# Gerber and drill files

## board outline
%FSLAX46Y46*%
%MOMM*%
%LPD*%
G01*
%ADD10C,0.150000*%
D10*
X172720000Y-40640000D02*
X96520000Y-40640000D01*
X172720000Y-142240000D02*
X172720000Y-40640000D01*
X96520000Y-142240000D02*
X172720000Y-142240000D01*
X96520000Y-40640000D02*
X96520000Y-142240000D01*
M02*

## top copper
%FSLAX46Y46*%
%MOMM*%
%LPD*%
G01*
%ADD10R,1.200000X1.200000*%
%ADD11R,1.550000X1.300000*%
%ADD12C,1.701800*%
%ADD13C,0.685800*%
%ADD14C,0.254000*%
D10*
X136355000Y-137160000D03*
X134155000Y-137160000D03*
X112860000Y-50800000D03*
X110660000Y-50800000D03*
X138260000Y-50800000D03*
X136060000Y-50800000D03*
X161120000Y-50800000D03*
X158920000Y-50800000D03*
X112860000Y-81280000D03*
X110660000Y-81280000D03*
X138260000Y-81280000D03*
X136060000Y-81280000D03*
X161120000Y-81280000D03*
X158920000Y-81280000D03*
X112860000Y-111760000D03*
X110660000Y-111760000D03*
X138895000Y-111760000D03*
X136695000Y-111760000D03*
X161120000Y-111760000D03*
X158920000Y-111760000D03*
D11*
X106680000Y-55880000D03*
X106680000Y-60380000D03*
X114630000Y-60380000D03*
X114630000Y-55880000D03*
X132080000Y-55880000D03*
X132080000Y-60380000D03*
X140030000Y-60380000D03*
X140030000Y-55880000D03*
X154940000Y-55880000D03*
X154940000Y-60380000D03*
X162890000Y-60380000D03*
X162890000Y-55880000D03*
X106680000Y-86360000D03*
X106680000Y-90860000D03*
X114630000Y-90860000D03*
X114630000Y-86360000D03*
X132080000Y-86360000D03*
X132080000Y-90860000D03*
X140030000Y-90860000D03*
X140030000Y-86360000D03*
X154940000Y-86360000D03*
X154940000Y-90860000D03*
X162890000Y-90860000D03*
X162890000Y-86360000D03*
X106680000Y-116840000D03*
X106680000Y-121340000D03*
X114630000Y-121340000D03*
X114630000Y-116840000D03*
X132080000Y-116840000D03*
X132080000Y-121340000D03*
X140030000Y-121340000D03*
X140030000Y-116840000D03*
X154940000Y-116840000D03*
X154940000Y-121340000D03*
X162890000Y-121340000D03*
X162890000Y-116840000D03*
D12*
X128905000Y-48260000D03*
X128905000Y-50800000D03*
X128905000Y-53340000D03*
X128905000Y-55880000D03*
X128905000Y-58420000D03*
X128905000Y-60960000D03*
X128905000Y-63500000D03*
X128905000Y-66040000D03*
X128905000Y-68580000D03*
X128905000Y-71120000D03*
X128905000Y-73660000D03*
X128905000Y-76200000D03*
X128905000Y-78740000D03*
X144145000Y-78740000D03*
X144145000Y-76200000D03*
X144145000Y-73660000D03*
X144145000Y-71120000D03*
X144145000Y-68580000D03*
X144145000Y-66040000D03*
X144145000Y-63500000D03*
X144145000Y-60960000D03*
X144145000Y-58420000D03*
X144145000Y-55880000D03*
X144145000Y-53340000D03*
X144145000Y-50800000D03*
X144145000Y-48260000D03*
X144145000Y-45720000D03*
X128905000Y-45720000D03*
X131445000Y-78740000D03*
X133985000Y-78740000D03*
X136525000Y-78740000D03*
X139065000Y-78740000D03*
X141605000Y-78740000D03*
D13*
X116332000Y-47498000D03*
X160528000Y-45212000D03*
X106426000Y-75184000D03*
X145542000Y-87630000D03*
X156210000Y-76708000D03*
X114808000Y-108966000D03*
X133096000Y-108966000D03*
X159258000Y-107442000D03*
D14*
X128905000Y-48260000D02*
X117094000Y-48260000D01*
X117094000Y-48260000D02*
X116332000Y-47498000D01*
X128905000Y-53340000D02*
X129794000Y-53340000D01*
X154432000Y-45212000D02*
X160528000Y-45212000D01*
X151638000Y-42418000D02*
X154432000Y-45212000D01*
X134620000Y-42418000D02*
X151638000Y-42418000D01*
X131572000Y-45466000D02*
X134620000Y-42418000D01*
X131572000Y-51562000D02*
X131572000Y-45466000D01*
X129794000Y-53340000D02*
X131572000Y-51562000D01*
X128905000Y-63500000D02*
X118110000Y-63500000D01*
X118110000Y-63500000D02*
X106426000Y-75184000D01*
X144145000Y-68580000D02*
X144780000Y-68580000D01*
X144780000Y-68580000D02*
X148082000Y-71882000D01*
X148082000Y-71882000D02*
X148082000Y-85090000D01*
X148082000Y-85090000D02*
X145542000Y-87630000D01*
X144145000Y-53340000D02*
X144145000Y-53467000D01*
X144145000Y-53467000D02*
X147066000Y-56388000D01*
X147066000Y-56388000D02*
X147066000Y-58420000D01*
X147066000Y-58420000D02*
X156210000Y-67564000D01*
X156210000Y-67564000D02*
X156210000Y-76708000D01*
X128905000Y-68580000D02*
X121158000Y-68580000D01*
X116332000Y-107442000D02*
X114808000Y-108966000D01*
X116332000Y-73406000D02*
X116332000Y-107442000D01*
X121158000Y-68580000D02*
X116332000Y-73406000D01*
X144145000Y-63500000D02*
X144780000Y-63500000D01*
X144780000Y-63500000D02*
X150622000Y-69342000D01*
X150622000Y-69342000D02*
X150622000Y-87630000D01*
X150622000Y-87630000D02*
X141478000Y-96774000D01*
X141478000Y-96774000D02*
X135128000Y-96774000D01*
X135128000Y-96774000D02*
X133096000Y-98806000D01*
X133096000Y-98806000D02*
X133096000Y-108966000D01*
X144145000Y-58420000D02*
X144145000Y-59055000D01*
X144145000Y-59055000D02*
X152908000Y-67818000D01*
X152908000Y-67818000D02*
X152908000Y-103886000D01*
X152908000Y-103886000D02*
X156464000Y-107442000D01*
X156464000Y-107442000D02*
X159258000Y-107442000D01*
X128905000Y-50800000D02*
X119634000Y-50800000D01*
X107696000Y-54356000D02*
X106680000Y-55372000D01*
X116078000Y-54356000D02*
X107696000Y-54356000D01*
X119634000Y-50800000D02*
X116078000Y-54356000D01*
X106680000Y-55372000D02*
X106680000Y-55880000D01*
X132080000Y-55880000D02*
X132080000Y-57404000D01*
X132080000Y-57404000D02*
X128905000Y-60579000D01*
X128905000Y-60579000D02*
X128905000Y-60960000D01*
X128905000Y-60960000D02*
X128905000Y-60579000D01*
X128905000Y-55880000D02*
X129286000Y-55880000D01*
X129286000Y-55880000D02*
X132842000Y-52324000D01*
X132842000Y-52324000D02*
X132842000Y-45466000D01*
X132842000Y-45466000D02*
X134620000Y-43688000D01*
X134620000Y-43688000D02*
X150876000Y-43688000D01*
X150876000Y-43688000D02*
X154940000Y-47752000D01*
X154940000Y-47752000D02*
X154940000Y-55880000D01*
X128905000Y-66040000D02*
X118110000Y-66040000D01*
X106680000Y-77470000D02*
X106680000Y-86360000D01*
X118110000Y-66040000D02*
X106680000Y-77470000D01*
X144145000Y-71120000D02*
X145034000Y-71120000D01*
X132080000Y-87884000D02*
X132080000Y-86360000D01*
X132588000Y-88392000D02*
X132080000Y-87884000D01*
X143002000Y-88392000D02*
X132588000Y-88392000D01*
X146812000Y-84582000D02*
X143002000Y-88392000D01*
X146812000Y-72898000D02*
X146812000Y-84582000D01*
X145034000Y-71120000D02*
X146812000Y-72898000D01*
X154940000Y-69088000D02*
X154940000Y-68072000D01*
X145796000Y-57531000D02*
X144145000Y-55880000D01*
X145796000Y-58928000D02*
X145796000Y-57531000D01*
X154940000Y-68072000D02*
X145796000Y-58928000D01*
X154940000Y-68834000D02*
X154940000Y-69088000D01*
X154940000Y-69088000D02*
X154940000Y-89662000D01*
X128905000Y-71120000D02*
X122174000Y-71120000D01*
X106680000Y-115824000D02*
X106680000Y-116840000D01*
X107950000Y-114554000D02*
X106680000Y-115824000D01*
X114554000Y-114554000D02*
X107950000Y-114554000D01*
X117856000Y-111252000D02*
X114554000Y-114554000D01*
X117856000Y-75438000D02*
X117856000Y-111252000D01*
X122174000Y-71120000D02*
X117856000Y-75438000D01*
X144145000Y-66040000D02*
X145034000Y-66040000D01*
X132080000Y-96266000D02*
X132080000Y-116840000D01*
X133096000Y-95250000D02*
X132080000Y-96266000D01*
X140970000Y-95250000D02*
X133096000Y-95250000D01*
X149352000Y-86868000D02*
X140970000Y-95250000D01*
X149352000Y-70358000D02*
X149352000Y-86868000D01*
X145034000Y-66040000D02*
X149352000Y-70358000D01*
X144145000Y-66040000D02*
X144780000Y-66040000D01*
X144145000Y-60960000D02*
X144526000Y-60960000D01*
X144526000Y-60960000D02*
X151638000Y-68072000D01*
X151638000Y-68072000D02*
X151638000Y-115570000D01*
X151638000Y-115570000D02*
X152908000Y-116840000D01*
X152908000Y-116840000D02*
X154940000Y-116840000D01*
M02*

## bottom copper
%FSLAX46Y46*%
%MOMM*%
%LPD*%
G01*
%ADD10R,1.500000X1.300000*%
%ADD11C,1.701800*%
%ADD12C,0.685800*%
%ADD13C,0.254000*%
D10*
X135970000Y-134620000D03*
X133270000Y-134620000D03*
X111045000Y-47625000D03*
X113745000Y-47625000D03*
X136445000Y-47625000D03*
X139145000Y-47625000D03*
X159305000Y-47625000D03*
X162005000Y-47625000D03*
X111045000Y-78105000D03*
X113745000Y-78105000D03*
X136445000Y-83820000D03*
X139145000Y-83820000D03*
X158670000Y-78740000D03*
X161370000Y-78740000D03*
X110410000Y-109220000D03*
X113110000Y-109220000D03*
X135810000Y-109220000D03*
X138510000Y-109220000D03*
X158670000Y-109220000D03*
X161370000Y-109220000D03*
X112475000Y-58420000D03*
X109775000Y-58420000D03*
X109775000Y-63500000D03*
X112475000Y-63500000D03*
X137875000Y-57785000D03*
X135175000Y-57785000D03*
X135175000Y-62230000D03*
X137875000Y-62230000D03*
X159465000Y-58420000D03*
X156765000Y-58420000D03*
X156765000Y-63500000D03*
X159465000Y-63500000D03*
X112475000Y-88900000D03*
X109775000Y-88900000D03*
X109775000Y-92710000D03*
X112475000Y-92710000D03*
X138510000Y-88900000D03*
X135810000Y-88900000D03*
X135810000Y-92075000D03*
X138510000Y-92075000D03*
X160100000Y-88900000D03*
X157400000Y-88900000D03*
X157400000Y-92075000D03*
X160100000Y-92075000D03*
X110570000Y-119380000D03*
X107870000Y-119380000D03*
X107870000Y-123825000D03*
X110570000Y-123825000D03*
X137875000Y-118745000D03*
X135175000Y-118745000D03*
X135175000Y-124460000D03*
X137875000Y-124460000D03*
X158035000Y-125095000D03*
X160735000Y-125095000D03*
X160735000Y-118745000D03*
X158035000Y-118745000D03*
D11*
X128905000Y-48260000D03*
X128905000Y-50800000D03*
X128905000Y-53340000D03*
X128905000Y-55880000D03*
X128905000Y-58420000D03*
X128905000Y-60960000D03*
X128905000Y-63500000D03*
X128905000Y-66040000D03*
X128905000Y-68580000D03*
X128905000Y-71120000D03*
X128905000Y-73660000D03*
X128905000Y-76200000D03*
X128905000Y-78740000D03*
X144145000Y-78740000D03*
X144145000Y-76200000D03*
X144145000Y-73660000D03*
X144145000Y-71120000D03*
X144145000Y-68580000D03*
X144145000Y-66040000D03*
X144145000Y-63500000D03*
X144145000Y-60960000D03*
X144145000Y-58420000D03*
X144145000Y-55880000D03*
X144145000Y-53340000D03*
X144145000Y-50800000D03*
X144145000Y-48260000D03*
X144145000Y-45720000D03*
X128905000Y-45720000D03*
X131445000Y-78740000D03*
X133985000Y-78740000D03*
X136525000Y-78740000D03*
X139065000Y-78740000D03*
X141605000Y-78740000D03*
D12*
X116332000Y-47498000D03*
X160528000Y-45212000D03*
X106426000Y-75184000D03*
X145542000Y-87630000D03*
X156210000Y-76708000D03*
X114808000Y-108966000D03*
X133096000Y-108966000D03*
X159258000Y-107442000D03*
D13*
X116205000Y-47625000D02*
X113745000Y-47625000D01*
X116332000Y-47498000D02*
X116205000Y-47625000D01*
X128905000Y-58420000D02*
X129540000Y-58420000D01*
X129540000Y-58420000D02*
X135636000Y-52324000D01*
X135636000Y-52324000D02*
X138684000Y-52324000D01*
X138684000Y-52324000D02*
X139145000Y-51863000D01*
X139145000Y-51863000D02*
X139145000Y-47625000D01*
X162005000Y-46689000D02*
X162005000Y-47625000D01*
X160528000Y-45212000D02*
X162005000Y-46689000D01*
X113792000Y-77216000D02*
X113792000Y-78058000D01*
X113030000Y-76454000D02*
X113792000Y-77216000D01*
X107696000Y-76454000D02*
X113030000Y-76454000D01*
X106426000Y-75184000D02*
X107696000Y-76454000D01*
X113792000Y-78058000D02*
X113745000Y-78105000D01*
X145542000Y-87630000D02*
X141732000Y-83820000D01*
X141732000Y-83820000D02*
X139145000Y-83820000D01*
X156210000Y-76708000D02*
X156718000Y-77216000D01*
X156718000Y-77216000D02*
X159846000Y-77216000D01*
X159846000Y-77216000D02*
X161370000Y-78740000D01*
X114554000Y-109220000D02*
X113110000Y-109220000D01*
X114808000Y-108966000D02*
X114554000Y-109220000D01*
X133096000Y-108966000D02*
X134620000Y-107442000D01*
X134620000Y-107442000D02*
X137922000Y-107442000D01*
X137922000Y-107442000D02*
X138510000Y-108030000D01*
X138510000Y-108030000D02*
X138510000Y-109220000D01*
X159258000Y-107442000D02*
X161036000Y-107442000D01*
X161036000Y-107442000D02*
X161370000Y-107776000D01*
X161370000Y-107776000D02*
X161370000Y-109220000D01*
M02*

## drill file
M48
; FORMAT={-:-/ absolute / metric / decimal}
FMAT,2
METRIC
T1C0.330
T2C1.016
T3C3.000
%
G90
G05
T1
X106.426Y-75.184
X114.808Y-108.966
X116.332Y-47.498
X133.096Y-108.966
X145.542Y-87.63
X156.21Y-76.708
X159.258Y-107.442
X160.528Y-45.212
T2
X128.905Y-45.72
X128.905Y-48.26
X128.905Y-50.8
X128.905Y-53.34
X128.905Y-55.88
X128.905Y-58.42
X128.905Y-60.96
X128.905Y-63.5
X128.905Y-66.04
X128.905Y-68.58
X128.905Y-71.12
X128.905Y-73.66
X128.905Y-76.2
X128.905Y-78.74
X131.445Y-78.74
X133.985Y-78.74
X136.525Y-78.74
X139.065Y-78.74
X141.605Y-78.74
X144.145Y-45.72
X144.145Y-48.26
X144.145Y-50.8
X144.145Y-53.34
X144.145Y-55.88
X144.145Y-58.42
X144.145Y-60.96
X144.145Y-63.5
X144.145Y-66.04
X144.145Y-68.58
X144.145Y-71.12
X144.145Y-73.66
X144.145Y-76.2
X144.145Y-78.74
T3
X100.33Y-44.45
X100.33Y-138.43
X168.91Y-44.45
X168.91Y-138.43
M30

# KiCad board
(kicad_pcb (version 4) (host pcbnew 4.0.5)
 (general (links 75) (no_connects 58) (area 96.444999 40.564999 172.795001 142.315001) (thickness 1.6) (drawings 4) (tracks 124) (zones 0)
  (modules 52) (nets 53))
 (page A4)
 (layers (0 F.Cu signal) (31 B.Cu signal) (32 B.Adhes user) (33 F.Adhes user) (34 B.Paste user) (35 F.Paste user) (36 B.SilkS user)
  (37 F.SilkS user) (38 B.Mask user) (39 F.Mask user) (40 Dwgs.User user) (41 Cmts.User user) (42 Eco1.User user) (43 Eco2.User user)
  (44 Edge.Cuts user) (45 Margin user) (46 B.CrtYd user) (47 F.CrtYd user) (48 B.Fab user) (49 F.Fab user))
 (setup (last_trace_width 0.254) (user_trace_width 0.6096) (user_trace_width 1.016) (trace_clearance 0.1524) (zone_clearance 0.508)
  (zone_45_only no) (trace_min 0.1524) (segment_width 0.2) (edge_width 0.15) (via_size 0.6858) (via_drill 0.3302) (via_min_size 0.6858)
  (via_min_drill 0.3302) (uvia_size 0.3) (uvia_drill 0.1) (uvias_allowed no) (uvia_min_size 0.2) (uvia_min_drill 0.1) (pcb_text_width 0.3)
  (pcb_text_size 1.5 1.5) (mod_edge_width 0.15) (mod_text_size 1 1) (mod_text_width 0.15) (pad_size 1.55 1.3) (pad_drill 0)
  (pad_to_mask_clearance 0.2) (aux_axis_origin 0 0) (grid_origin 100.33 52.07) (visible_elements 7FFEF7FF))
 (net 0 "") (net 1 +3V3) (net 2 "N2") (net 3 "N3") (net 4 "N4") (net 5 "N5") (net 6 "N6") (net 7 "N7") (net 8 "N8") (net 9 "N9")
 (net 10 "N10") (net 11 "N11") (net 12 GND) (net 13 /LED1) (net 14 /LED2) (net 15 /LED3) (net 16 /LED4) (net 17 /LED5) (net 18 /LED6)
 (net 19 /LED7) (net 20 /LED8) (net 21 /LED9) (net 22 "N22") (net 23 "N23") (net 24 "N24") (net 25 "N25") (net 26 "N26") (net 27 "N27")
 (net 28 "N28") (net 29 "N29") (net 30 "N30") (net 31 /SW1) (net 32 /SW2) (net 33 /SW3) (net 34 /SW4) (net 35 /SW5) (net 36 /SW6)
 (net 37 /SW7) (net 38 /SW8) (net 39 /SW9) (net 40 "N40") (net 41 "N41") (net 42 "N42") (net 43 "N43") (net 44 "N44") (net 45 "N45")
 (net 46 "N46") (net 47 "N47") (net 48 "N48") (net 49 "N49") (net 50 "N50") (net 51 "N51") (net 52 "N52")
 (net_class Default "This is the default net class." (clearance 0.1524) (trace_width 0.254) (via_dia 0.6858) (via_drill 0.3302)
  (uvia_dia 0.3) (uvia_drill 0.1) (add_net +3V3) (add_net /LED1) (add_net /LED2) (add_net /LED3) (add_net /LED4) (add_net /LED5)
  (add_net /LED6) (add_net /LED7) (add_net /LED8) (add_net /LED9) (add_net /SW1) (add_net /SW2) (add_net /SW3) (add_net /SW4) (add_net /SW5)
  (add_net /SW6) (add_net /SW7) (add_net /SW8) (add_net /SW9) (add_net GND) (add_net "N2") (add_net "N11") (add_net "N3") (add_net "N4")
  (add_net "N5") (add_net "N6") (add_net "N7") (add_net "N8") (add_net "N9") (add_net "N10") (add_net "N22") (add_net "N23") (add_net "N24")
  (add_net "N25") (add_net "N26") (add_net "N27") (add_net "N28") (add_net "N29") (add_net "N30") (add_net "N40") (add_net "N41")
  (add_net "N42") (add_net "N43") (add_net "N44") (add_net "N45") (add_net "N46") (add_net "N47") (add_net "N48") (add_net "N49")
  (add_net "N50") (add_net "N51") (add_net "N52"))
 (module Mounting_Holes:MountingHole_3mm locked (layer F.Cu) (at 168.91 138.43)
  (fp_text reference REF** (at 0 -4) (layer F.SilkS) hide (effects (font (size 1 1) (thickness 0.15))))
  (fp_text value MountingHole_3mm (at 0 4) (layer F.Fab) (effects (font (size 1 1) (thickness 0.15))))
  (pad 1 np_thru_hole circle (at 0 0) (size 3 3) (drill 3) (layers *.Cu *.Mask)))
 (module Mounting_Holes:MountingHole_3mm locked (layer F.Cu) (at 100.33 138.43)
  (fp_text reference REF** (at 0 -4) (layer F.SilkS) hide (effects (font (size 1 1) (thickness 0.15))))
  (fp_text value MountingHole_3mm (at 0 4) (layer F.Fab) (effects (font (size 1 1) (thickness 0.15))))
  (pad 1 np_thru_hole circle (at 0 0) (size 3 3) (drill 3) (layers *.Cu *.Mask)))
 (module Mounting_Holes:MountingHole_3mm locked (layer F.Cu) (at 100.33 44.45)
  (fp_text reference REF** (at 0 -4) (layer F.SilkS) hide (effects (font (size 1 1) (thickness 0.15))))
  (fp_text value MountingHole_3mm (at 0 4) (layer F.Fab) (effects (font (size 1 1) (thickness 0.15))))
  (pad 1 np_thru_hole circle (at 0 0) (size 3 3) (drill 3) (layers *.Cu *.Mask)))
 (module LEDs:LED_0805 (layer F.Cu) (at 135.255 137.16)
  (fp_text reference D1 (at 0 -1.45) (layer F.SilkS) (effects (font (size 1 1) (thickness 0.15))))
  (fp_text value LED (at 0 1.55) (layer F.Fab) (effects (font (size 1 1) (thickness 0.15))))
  (pad 2 smd rect (at 1.1 0 180) (size 1.2 1.2) (layers F.Cu F.Paste F.Mask) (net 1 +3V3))
  (pad 1 smd rect (at -1.1 0 180) (size 1.2 1.2) (layers F.Cu F.Paste F.Mask) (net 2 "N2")))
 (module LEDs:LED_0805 (layer F.Cu) (at 111.76 50.8)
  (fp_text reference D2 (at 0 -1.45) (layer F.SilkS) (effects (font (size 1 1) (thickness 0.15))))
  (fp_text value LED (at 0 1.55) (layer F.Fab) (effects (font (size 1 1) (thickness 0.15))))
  (pad 2 smd rect (at 1.1 0 180) (size 1.2 1.2) (layers F.Cu F.Paste F.Mask) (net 1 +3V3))
  (pad 1 smd rect (at -1.1 0 180) (size 1.2 1.2) (layers F.Cu F.Paste F.Mask) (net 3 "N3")))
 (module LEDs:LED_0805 (layer F.Cu) (at 137.16 50.8)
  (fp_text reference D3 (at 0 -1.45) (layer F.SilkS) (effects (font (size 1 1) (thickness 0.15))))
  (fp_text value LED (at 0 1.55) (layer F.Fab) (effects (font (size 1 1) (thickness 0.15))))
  (pad 2 smd rect (at 1.1 0 180) (size 1.2 1.2) (layers F.Cu F.Paste F.Mask) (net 1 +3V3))
  (pad 1 smd rect (at -1.1 0 180) (size 1.2 1.2) (layers F.Cu F.Paste F.Mask) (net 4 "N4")))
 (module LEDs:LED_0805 (layer F.Cu) (at 160.02 50.8)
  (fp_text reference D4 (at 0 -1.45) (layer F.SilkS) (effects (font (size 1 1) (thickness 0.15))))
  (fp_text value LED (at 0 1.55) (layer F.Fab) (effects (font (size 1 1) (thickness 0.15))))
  (pad 2 smd rect (at 1.1 0 180) (size 1.2 1.2) (layers F.Cu F.Paste F.Mask) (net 1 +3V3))
  (pad 1 smd rect (at -1.1 0 180) (size 1.2 1.2) (layers F.Cu F.Paste F.Mask) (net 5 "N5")))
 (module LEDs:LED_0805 (layer F.Cu) (at 111.76 81.28)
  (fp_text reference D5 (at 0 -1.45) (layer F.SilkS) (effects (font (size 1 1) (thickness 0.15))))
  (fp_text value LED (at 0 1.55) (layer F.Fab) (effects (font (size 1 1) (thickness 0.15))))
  (pad 2 smd rect (at 1.1 0 180) (size 1.2 1.2) (layers F.Cu F.Paste F.Mask) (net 1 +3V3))
  (pad 1 smd rect (at -1.1 0 180) (size 1.2 1.2) (layers F.Cu F.Paste F.Mask) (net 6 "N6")))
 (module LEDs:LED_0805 (layer F.Cu) (at 137.16 81.28)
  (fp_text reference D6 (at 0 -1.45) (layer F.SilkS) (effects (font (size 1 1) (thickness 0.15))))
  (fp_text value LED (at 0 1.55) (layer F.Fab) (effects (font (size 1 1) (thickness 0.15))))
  (pad 2 smd rect (at 1.1 0 180) (size 1.2 1.2) (layers F.Cu F.Paste F.Mask) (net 1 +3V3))
  (pad 1 smd rect (at -1.1 0 180) (size 1.2 1.2) (layers F.Cu F.Paste F.Mask) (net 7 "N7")))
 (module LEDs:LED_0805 (layer F.Cu) (at 160.02 81.28)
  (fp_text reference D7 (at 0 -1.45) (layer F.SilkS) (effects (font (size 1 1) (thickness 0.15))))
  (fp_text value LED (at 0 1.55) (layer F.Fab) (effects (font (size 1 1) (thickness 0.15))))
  (pad 2 smd rect (at 1.1 0 180) (size 1.2 1.2) (layers F.Cu F.Paste F.Mask) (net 1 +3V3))
  (pad 1 smd rect (at -1.1 0 180) (size 1.2 1.2) (layers F.Cu F.Paste F.Mask) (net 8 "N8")))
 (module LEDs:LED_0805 (layer F.Cu) (at 111.76 111.76)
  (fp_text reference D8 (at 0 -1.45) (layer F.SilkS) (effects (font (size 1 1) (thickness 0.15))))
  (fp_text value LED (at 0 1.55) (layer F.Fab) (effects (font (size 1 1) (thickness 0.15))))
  (pad 2 smd rect (at 1.1 0 180) (size 1.2 1.2) (layers F.Cu F.Paste F.Mask) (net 1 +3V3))
  (pad 1 smd rect (at -1.1 0 180) (size 1.2 1.2) (layers F.Cu F.Paste F.Mask) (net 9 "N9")))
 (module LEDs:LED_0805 (layer F.Cu) (at 137.795 111.76)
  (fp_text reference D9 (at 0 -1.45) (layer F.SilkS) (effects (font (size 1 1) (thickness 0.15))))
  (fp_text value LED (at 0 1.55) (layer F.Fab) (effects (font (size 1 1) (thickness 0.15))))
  (pad 2 smd rect (at 1.1 0 180) (size 1.2 1.2) (layers F.Cu F.Paste F.Mask) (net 1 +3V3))
  (pad 1 smd rect (at -1.1 0 180) (size 1.2 1.2) (layers F.Cu F.Paste F.Mask) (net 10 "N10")))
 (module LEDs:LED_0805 (layer F.Cu) (at 160.02 111.76)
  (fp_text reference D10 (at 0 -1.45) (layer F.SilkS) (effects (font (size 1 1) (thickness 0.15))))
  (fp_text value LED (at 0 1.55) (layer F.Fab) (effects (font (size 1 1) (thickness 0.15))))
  (pad 2 smd rect (at 1.1 0 180) (size 1.2 1.2) (layers F.Cu F.Paste F.Mask) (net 1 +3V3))
  (pad 1 smd rect (at -1.1 0 180) (size 1.2 1.2) (layers F.Cu F.Paste F.Mask) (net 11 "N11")))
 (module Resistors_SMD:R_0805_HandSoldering (layer B.Cu) (at 134.62 134.62 180)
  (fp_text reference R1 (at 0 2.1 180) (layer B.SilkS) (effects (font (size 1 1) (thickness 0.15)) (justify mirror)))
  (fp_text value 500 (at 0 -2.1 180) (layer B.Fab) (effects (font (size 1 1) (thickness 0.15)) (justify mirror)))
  (pad 1 smd rect (at -1.35 0 180) (size 1.5 1.3) (layers B.Cu B.Paste B.Mask) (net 2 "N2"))
  (pad 2 smd rect (at 1.35 0 180) (size 1.5 1.3) (layers B.Cu B.Paste B.Mask) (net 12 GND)))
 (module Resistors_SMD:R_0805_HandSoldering (layer B.Cu) (at 112.395 47.625)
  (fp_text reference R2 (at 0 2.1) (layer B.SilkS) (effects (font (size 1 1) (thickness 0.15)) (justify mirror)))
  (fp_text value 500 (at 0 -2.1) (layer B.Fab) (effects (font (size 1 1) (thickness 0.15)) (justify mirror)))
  (pad 1 smd rect (at -1.35 0) (size 1.5 1.3) (layers B.Cu B.Paste B.Mask) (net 3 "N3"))
  (pad 2 smd rect (at 1.35 0) (size 1.5 1.3) (layers B.Cu B.Paste B.Mask) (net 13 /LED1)))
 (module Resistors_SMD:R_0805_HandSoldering (layer B.Cu) (at 137.795 47.625)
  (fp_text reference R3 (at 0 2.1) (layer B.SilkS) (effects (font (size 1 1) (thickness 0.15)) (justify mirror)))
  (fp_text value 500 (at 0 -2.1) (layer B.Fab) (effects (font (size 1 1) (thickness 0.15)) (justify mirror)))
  (pad 1 smd rect (at -1.35 0) (size 1.5 1.3) (layers B.Cu B.Paste B.Mask) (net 4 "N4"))
  (pad 2 smd rect (at 1.35 0) (size 1.5 1.3) (layers B.Cu B.Paste B.Mask) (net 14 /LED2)))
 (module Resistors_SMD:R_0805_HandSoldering (layer B.Cu) (at 160.655 47.625)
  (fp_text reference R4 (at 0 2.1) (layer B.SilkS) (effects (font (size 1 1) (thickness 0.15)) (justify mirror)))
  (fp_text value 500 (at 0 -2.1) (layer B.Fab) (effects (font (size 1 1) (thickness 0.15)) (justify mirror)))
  (pad 1 smd rect (at -1.35 0) (size 1.5 1.3) (layers B.Cu B.Paste B.Mask) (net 5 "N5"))
  (pad 2 smd rect (at 1.35 0) (size 1.5 1.3) (layers B.Cu B.Paste B.Mask) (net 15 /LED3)))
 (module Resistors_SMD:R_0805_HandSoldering (layer B.Cu) (at 112.395 78.105)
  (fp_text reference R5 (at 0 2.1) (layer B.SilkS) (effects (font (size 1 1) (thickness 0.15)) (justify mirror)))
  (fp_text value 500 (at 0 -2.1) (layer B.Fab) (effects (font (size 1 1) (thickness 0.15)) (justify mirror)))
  (pad 1 smd rect (at -1.35 0) (size 1.5 1.3) (layers B.Cu B.Paste B.Mask) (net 6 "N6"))
  (pad 2 smd rect (at 1.35 0) (size 1.5 1.3) (layers B.Cu B.Paste B.Mask) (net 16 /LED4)))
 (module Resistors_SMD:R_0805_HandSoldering (layer B.Cu) (at 137.795 83.82)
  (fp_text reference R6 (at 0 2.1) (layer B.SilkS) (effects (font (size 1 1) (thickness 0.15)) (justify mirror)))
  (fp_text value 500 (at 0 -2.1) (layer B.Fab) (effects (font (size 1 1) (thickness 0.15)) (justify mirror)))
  (pad 1 smd rect (at -1.35 0) (size 1.5 1.3) (layers B.Cu B.Paste B.Mask) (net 7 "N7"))
  (pad 2 smd rect (at 1.35 0) (size 1.5 1.3) (layers B.Cu B.Paste B.Mask) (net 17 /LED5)))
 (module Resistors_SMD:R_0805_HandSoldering (layer B.Cu) (at 160.02 78.74)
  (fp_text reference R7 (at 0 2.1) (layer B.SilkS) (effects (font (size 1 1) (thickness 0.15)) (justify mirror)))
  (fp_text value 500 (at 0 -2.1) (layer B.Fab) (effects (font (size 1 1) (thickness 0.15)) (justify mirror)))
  (pad 1 smd rect (at -1.35 0) (size 1.5 1.3) (layers B.Cu B.Paste B.Mask) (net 8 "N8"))
  (pad 2 smd rect (at 1.35 0) (size 1.5 1.3) (layers B.Cu B.Paste B.Mask) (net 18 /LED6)))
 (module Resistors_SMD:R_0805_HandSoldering (layer B.Cu) (at 111.76 109.22)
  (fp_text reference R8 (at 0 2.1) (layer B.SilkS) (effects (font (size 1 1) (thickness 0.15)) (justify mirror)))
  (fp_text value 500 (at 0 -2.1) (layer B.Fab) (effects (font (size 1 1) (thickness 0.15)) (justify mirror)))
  (pad 1 smd rect (at -1.35 0) (size 1.5 1.3) (layers B.Cu B.Paste B.Mask) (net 9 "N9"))
  (pad 2 smd rect (at 1.35 0) (size 1.5 1.3) (layers B.Cu B.Paste B.Mask) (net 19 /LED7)))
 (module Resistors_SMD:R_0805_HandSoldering (layer B.Cu) (at 137.16 109.22)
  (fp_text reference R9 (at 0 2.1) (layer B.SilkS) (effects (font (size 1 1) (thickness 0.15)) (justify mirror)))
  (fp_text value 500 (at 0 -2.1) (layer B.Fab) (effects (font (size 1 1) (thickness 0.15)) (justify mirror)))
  (pad 1 smd rect (at -1.35 0) (size 1.5 1.3) (layers B.Cu B.Paste B.Mask) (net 10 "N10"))
  (pad 2 smd rect (at 1.35 0) (size 1.5 1.3) (layers B.Cu B.Paste B.Mask) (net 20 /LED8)))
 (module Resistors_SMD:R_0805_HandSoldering (layer B.Cu) (at 160.02 109.22)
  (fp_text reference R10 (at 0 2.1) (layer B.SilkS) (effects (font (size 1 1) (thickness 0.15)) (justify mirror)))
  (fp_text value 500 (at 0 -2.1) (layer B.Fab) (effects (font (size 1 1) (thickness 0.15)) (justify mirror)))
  (pad 1 smd rect (at -1.35 0) (size 1.5 1.3) (layers B.Cu B.Paste B.Mask) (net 11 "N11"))
  (pad 2 smd rect (at 1.35 0) (size 1.5 1.3) (layers B.Cu B.Paste B.Mask) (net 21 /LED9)))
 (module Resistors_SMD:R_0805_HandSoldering (layer B.Cu) (at 111.125 58.42 180)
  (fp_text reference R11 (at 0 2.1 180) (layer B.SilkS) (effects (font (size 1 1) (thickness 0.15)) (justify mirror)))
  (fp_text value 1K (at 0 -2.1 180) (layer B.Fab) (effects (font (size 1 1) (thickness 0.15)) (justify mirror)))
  (pad 1 smd rect (at -1.35 0 180) (size 1.5 1.3) (layers B.Cu B.Paste B.Mask) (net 1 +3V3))
  (pad 2 smd rect (at 1.35 0 180) (size 1.5 1.3) (layers B.Cu B.Paste B.Mask) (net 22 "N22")))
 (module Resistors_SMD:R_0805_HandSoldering (layer B.Cu) (at 111.125 63.5)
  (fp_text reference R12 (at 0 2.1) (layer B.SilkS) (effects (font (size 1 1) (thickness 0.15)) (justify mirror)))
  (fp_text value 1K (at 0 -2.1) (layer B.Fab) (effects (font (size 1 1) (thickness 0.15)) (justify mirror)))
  (pad 1 smd rect (at -1.35 0) (size 1.5 1.3) (layers B.Cu B.Paste B.Mask) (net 22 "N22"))
  (pad 2 smd rect (at 1.35 0) (size 1.5 1.3) (layers B.Cu B.Paste B.Mask) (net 12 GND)))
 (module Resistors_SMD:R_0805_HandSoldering (layer B.Cu) (at 136.525 57.785 180)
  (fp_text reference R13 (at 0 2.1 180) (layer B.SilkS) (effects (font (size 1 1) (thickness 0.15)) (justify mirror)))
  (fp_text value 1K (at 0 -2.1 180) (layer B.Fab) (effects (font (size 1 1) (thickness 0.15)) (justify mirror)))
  (pad 1 smd rect (at -1.35 0 180) (size 1.5 1.3) (layers B.Cu B.Paste B.Mask) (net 1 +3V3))
  (pad 2 smd rect (at 1.35 0 180) (size 1.5 1.3) (layers B.Cu B.Paste B.Mask) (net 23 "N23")))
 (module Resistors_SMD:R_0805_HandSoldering (layer B.Cu) (at 136.525 62.23)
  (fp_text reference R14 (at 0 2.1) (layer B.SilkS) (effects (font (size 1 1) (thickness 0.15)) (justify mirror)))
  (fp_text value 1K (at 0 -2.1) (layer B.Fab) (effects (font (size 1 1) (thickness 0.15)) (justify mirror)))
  (pad 1 smd rect (at -1.35 0) (size 1.5 1.3) (layers B.Cu B.Paste B.Mask) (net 23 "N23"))
  (pad 2 smd rect (at 1.35 0) (size 1.5 1.3) (layers B.Cu B.Paste B.Mask) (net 12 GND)))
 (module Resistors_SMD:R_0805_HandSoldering (layer B.Cu) (at 158.115 58.42 180)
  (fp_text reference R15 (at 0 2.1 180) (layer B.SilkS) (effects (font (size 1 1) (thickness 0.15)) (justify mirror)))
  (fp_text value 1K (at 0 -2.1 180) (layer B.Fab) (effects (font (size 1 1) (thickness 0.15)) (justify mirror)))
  (pad 1 smd rect (at -1.35 0 180) (size 1.5 1.3) (layers B.Cu B.Paste B.Mask) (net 1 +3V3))
  (pad 2 smd rect (at 1.35 0 180) (size 1.5 1.3) (layers B.Cu B.Paste B.Mask) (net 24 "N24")))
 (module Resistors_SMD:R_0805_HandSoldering (layer B.Cu) (at 158.115 63.5)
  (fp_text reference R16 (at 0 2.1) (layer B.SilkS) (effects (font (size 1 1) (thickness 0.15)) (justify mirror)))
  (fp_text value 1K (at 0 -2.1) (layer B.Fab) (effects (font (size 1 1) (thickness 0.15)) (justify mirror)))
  (pad 1 smd rect (at -1.35 0) (size 1.5 1.3) (layers B.Cu B.Paste B.Mask) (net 24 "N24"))
  (pad 2 smd rect (at 1.35 0) (size 1.5 1.3) (layers B.Cu B.Paste B.Mask) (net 12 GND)))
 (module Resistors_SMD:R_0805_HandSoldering (layer B.Cu) (at 111.125 88.9 180)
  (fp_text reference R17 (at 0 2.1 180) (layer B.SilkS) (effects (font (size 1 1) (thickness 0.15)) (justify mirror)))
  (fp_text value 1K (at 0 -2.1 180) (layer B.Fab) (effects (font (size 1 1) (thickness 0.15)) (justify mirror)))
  (pad 1 smd rect (at -1.35 0 180) (size 1.5 1.3) (layers B.Cu B.Paste B.Mask) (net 1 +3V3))
  (pad 2 smd rect (at 1.35 0 180) (size 1.5 1.3) (layers B.Cu B.Paste B.Mask) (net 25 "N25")))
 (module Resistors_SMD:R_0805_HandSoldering (layer B.Cu) (at 111.125 92.71)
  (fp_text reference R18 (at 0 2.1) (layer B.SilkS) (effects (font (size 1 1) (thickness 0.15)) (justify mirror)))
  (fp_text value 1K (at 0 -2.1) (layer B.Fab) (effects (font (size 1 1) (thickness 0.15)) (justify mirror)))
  (pad 1 smd rect (at -1.35 0) (size 1.5 1.3) (layers B.Cu B.Paste B.Mask) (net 25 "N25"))
  (pad 2 smd rect (at 1.35 0) (size 1.5 1.3) (layers B.Cu B.Paste B.Mask) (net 12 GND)))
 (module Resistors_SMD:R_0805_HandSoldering (layer B.Cu) (at 137.16 88.9 180)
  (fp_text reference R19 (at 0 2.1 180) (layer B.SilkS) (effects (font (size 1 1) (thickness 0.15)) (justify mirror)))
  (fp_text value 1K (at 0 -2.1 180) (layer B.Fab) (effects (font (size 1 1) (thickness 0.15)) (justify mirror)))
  (pad 1 smd rect (at -1.35 0 180) (size 1.5 1.3) (layers B.Cu B.Paste B.Mask) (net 1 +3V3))
  (pad 2 smd rect (at 1.35 0 180) (size 1.5 1.3) (layers B.Cu B.Paste B.Mask) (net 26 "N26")))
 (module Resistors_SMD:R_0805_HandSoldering (layer B.Cu) (at 137.16 92.075)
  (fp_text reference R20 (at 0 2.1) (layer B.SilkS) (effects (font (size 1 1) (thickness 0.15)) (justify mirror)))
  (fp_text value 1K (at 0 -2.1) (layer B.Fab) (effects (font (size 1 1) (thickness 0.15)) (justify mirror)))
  (pad 1 smd rect (at -1.35 0) (size 1.5 1.3) (layers B.Cu B.Paste B.Mask) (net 26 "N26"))
  (pad 2 smd rect (at 1.35 0) (size 1.5 1.3) (layers B.Cu B.Paste B.Mask) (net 12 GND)))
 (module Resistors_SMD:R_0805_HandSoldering (layer B.Cu) (at 158.75 88.9 180)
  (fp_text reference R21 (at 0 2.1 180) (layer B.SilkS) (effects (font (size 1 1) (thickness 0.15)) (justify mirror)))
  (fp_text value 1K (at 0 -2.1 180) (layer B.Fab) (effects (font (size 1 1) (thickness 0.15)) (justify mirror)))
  (pad 1 smd rect (at -1.35 0 180) (size 1.5 1.3) (layers B.Cu B.Paste B.Mask) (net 1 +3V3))
  (pad 2 smd rect (at 1.35 0 180) (size 1.5 1.3) (layers B.Cu B.Paste B.Mask) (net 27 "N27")))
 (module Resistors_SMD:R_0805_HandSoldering (layer B.Cu) (at 158.75 92.075)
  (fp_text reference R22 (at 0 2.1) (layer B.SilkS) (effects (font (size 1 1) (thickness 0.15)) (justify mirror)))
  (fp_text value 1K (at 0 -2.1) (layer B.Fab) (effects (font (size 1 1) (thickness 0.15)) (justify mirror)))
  (pad 1 smd rect (at -1.35 0) (size 1.5 1.3) (layers B.Cu B.Paste B.Mask) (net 27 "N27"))
  (pad 2 smd rect (at 1.35 0) (size 1.5 1.3) (layers B.Cu B.Paste B.Mask) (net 12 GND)))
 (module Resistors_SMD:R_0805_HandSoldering (layer B.Cu) (at 109.22 119.38 180)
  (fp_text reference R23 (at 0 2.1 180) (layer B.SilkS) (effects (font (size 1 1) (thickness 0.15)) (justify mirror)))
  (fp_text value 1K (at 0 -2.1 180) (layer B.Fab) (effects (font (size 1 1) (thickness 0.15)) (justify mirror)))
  (pad 1 smd rect (at -1.35 0 180) (size 1.5 1.3) (layers B.Cu B.Paste B.Mask) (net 1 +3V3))
  (pad 2 smd rect (at 1.35 0 180) (size 1.5 1.3) (layers B.Cu B.Paste B.Mask) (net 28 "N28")))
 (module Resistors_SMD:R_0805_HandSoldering (layer B.Cu) (at 109.22 123.825)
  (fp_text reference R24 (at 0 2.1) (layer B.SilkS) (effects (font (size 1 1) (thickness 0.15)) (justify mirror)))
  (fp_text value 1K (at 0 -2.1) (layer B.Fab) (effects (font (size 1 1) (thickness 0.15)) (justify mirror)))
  (pad 1 smd rect (at -1.35 0) (size 1.5 1.3) (layers B.Cu B.Paste B.Mask) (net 28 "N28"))
  (pad 2 smd rect (at 1.35 0) (size 1.5 1.3) (layers B.Cu B.Paste B.Mask) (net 12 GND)))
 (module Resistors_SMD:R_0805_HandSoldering (layer B.Cu) (at 136.525 118.745 180)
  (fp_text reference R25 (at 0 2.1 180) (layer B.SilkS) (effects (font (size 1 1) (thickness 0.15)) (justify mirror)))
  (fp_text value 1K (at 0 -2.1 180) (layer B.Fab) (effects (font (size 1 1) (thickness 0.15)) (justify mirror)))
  (pad 1 smd rect (at -1.35 0 180) (size 1.5 1.3) (layers B.Cu B.Paste B.Mask) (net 1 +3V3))
  (pad 2 smd rect (at 1.35 0 180) (size 1.5 1.3) (layers B.Cu B.Paste B.Mask) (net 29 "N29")))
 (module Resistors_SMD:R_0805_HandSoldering (layer B.Cu) (at 136.525 124.46)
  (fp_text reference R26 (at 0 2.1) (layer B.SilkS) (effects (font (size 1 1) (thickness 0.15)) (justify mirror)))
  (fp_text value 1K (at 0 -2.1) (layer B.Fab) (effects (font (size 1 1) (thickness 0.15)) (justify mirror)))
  (pad 1 smd rect (at -1.35 0) (size 1.5 1.3) (layers B.Cu B.Paste B.Mask) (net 29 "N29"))
  (pad 2 smd rect (at 1.35 0) (size 1.5 1.3) (layers B.Cu B.Paste B.Mask) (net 12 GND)))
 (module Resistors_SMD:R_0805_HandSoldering (layer B.Cu) (at 159.385 125.095)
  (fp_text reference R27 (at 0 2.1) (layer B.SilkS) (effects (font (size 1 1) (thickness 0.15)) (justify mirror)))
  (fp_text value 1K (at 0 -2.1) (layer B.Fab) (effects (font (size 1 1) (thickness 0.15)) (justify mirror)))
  (pad 1 smd rect (at -1.35 0) (size 1.5 1.3) (layers B.Cu B.Paste B.Mask) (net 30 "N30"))
  (pad 2 smd rect (at 1.35 0) (size 1.5 1.3) (layers B.Cu B.Paste B.Mask) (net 12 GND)))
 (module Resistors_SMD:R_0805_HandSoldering (layer B.Cu) (at 159.385 118.745 180)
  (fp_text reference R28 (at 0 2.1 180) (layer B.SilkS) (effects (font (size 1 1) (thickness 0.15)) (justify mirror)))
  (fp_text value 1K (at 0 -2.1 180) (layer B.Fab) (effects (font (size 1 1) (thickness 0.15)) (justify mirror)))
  (pad 1 smd rect (at -1.35 0 180) (size 1.5 1.3) (layers B.Cu B.Paste B.Mask) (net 1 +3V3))
  (pad 2 smd rect (at 1.35 0 180) (size 1.5 1.3) (layers B.Cu B.Paste B.Mask) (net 30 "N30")))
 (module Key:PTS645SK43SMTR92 (layer F.Cu) (at 106.68 55.88)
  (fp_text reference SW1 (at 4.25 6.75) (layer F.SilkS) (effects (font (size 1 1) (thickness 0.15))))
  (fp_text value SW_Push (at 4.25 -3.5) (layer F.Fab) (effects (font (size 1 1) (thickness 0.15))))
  (pad 1 smd rect (at 0 0) (size 1.55 1.3) (layers F.Cu F.Paste F.Mask) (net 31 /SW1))
  (pad 2 smd rect (at 0 4.5) (size 1.55 1.3) (layers F.Cu F.Paste F.Mask) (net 22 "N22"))
  (pad 3 smd rect (at 7.95 4.5) (size 1.55 1.3) (layers F.Cu F.Paste F.Mask))
  (pad 4 smd rect (at 7.95 0) (size 1.55 1.3) (layers F.Cu F.Paste F.Mask)))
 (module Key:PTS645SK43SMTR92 (layer F.Cu) (at 132.08 55.88)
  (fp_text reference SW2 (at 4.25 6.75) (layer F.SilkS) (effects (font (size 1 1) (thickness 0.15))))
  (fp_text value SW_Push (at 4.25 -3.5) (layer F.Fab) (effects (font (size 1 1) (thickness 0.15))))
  (pad 1 smd rect (at 0 0) (size 1.55 1.3) (layers F.Cu F.Paste F.Mask) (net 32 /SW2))
  (pad 2 smd rect (at 0 4.5) (size 1.55 1.3) (layers F.Cu F.Paste F.Mask) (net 23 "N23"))
  (pad 3 smd rect (at 7.95 4.5) (size 1.55 1.3) (layers F.Cu F.Paste F.Mask))
  (pad 4 smd rect (at 7.95 0) (size 1.55 1.3) (layers F.Cu F.Paste F.Mask)))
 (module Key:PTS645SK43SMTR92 (layer F.Cu) (at 154.94 55.88)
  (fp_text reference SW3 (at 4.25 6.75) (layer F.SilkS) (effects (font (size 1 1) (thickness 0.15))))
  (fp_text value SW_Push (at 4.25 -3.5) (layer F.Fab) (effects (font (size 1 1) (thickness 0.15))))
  (pad 1 smd rect (at 0 0) (size 1.55 1.3) (layers F.Cu F.Paste F.Mask) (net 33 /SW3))
  (pad 2 smd rect (at 0 4.5) (size 1.55 1.3) (layers F.Cu F.Paste F.Mask) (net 24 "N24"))
  (pad 3 smd rect (at 7.95 4.5) (size 1.55 1.3) (layers F.Cu F.Paste F.Mask))
  (pad 4 smd rect (at 7.95 0) (size 1.55 1.3) (layers F.Cu F.Paste F.Mask)))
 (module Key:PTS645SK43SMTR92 (layer F.Cu) (at 106.68 86.36)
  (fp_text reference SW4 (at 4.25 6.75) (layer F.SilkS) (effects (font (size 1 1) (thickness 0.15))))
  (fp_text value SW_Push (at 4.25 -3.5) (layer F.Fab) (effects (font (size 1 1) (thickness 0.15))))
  (pad 1 smd rect (at 0 0) (size 1.55 1.3) (layers F.Cu F.Paste F.Mask) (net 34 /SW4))
  (pad 2 smd rect (at 0 4.5) (size 1.55 1.3) (layers F.Cu F.Paste F.Mask) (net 25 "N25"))
  (pad 3 smd rect (at 7.95 4.5) (size 1.55 1.3) (layers F.Cu F.Paste F.Mask))
  (pad 4 smd rect (at 7.95 0) (size 1.55 1.3) (layers F.Cu F.Paste F.Mask)))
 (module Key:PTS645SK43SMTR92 (layer F.Cu) (at 132.08 86.36)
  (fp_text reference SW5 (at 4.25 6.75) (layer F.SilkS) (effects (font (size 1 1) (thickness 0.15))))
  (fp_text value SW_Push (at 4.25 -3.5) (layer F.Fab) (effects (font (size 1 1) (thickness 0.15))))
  (pad 1 smd rect (at 0 0) (size 1.55 1.3) (layers F.Cu F.Paste F.Mask) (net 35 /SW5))
  (pad 2 smd rect (at 0 4.5) (size 1.55 1.3) (layers F.Cu F.Paste F.Mask) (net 26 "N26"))
  (pad 3 smd rect (at 7.95 4.5) (size 1.55 1.3) (layers F.Cu F.Paste F.Mask))
  (pad 4 smd rect (at 7.95 0) (size 1.55 1.3) (layers F.Cu F.Paste F.Mask)))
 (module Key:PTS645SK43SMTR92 (layer F.Cu) (at 154.94 86.36)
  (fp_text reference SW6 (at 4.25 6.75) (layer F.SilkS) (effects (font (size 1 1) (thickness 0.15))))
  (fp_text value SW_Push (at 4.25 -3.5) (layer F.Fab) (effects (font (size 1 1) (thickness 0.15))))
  (pad 1 smd rect (at 0 0) (size 1.55 1.3) (layers F.Cu F.Paste F.Mask) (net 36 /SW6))
  (pad 2 smd rect (at 0 4.5) (size 1.55 1.3) (layers F.Cu F.Paste F.Mask) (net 27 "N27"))
  (pad 3 smd rect (at 7.95 4.5) (size 1.55 1.3) (layers F.Cu F.Paste F.Mask))
  (pad 4 smd rect (at 7.95 0) (size 1.55 1.3) (layers F.Cu F.Paste F.Mask)))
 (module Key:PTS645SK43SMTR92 (layer F.Cu) (at 106.68 116.84)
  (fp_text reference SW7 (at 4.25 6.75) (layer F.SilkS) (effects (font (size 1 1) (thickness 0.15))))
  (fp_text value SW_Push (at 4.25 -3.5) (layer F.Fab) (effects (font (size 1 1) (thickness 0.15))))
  (pad 1 smd rect (at 0 0) (size 1.55 1.3) (layers F.Cu F.Paste F.Mask) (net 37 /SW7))
  (pad 2 smd rect (at 0 4.5) (size 1.55 1.3) (layers F.Cu F.Paste F.Mask) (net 28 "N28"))
  (pad 3 smd rect (at 7.95 4.5) (size 1.55 1.3) (layers F.Cu F.Paste F.Mask))
  (pad 4 smd rect (at 7.95 0) (size 1.55 1.3) (layers F.Cu F.Paste F.Mask)))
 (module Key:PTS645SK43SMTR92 (layer F.Cu) (at 132.08 116.84)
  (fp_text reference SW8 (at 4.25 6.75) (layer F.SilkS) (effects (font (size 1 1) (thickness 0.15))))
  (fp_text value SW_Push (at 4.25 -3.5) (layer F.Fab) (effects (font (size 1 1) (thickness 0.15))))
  (pad 1 smd rect (at 0 0) (size 1.55 1.3) (layers F.Cu F.Paste F.Mask) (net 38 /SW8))
  (pad 2 smd rect (at 0 4.5) (size 1.55 1.3) (layers F.Cu F.Paste F.Mask) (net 29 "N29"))
  (pad 3 smd rect (at 7.95 4.5) (size 1.55 1.3) (layers F.Cu F.Paste F.Mask))
  (pad 4 smd rect (at 7.95 0) (size 1.55 1.3) (layers F.Cu F.Paste F.Mask)))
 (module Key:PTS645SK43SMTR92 (layer F.Cu) (at 154.94 116.84)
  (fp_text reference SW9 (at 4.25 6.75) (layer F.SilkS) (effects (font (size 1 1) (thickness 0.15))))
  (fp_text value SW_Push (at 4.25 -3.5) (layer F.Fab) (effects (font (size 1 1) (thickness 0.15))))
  (pad 1 smd rect (at 0 0) (size 1.55 1.3) (layers F.Cu F.Paste F.Mask) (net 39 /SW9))
  (pad 2 smd rect (at 0 4.5) (size 1.55 1.3) (layers F.Cu F.Paste F.Mask) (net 30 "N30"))
  (pad 3 smd rect (at 7.95 4.5) (size 1.55 1.3) (layers F.Cu F.Paste F.Mask))
  (pad 4 smd rect (at 7.95 0) (size 1.55 1.3) (layers F.Cu F.Paste F.Mask)))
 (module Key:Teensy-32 (layer B.Cu) (at 136.525 60.96 180)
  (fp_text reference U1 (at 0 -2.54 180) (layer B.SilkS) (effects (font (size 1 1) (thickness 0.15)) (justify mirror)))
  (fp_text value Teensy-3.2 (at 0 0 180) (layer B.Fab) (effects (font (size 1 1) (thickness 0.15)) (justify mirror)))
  (pad 0 thru_hole circle (at 7.62 12.7 180) (size 1.7018 1.7018) (drill 1.016) (layers *.Cu *.Mask) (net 13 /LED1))
  (pad 1 thru_hole circle (at 7.62 10.16 180) (size 1.7018 1.7018) (drill 1.016) (layers *.Cu *.Mask) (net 31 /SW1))
  (pad 2 thru_hole circle (at 7.62 7.62 180) (size 1.7018 1.7018) (drill 1.016) (layers *.Cu *.Mask) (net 15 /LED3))
  (pad 3 thru_hole circle (at 7.62 5.08 180) (size 1.7018 1.7018) (drill 1.016) (layers *.Cu *.Mask) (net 33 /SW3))
  (pad 4 thru_hole circle (at 7.62 2.54 180) (size 1.7018 1.7018) (drill 1.016) (layers *.Cu *.Mask) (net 14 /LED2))
  (pad 5 thru_hole circle (at 7.62 0 180) (size 1.7018 1.7018) (drill 1.016) (layers *.Cu *.Mask) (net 32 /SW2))
  (pad 6 thru_hole circle (at 7.62 -2.54 180) (size 1.7018 1.7018) (drill 1.016) (layers *.Cu *.Mask) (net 16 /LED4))
  (pad 7 thru_hole circle (at 7.62 -5.08 180) (size 1.7018 1.7018) (drill 1.016) (layers *.Cu *.Mask) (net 34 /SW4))
  (pad 8 thru_hole circle (at 7.62 -7.62 180) (size 1.7018 1.7018) (drill 1.016) (layers *.Cu *.Mask) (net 19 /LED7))
  (pad 9 thru_hole circle (at 7.62 -10.16 180) (size 1.7018 1.7018) (drill 1.016) (layers *.Cu *.Mask) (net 37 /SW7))
  (pad 10 thru_hole circle (at 7.62 -12.7 180) (size 1.7018 1.7018) (drill 1.016) (layers *.Cu *.Mask) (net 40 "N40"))
  (pad 11 thru_hole circle (at 7.62 -15.24 180) (size 1.7018 1.7018) (drill 1.016) (layers *.Cu *.Mask) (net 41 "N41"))
  (pad 12 thru_hole circle (at 7.62 -17.78 180) (size 1.7018 1.7018) (drill 1.016) (layers *.Cu *.Mask) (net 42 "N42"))
  (pad 13 thru_hole circle (at -7.62 -17.78 180) (size 1.7018 1.7018) (drill 1.016) (layers *.Cu *.Mask) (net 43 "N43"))
  (pad 14 thru_hole circle (at -7.62 -15.24 180) (size 1.7018 1.7018) (drill 1.016) (layers *.Cu *.Mask) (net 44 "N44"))
  (pad 15 thru_hole circle (at -7.62 -12.7 180) (size 1.7018 1.7018) (drill 1.016) (layers *.Cu *.Mask) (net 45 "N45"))
  (pad 16 thru_hole circle (at -7.62 -10.16 180) (size 1.7018 1.7018) (drill 1.016) (layers *.Cu *.Mask) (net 35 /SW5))
  (pad 17 thru_hole circle (at -7.62 -7.62 180) (size 1.7018 1.7018) (drill 1.016) (layers *.Cu *.Mask) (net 17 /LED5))
  (pad 18 thru_hole circle (at -7.62 -5.08 180) (size 1.7018 1.7018) (drill 1.016) (layers *.Cu *.Mask) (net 38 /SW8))
  (pad 19 thru_hole circle (at -7.62 -2.54 180) (size 1.7018 1.7018) (drill 1.016) (layers *.Cu *.Mask) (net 20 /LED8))
  (pad 20 thru_hole circle (at -7.62 0 180) (size 1.7018 1.7018) (drill 1.016) (layers *.Cu *.Mask) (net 39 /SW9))
  (pad 21 thru_hole circle (at -7.62 2.54 180) (size 1.7018 1.7018) (drill 1.016) (layers *.Cu *.Mask) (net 21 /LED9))
  (pad 22 thru_hole circle (at -7.62 5.08 180) (size 1.7018 1.7018) (drill 1.016) (layers *.Cu *.Mask) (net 36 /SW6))
  (pad 23 thru_hole circle (at -7.62 7.62 180) (size 1.7018 1.7018) (drill 1.016) (layers *.Cu *.Mask) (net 18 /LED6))
  (pad 24 thru_hole circle (at -7.62 10.16 180) (size 1.7018 1.7018) (drill 1.016) (layers *.Cu *.Mask) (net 1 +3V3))
  (pad 25 thru_hole circle (at -7.62 12.7 180) (size 1.7018 1.7018) (drill 1.016) (layers *.Cu *.Mask) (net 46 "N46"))
  (pad 26 thru_hole circle (at -7.62 15.24 180) (size 1.7018 1.7018) (drill 1.016) (layers *.Cu *.Mask) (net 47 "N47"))
  (pad 27 thru_hole circle (at 7.62 15.24 180) (size 1.7018 1.7018) (drill 1.016) (layers *.Cu *.Mask) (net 12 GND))
  (pad 28 thru_hole circle (at 5.08 -17.78 180) (size 1.7018 1.7018) (drill 1.016) (layers *.Cu *.Mask) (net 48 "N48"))
  (pad 29 thru_hole circle (at 2.54 -17.78 180) (size 1.7018 1.7018) (drill 1.016) (layers *.Cu *.Mask) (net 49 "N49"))
  (pad 30 thru_hole circle (at 0 -17.78 180) (size 1.7018 1.7018) (drill 1.016) (layers *.Cu *.Mask) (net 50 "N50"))
  (pad 31 thru_hole circle (at -2.54 -17.78 180) (size 1.7018 1.7018) (drill 1.016) (layers *.Cu *.Mask) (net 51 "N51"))
  (pad 32 thru_hole circle (at -5.08 -17.78 180) (size 1.7018 1.7018) (drill 1.016) (layers *.Cu *.Mask) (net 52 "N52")))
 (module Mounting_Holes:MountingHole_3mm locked (layer F.Cu) (at 168.91 44.45)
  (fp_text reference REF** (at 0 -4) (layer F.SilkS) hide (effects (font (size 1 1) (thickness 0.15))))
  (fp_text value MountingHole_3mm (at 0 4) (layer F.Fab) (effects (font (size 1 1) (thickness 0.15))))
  (pad 1 np_thru_hole circle (at 0 0) (size 3 3) (drill 3) (layers *.Cu *.Mask)))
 (gr_line (start 172.72 40.64) (end 96.52 40.64) (angle 90) (layer Edge.Cuts) (width 0.15))
 (gr_line (start 172.72 142.24) (end 172.72 40.64) (angle 90) (layer Edge.Cuts) (width 0.15))
 (gr_line (start 96.52 142.24) (end 172.72 142.24) (angle 90) (layer Edge.Cuts) (width 0.15))
 (gr_line (start 96.52 40.64) (end 96.52 142.24) (angle 90) (layer Edge.Cuts) (width 0.15))
 (segment (start 128.905 48.26) (end 117.094 48.26) (width 0.254) (layer F.Cu) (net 13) (status 400000))
 (segment (start 116.205 47.625) (end 113.745 47.625) (width 0.254) (layer B.Cu) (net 13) (status 800000))
 (segment (start 116.332 47.498) (end 116.205 47.625) (width 0.254) (layer B.Cu) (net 13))
 (via (at 116.332 47.498) (size 0.6858) (drill 0.3302) (layers F.Cu B.Cu) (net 13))
 (segment (start 117.094 48.26) (end 116.332 47.498) (width 0.254) (layer F.Cu) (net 13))
 (segment (start 128.905 58.42) (end 129.54 58.42) (width 0.254) (layer B.Cu) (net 14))
 (segment (start 129.54 58.42) (end 135.636 52.324) (width 0.254) (layer B.Cu) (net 14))
 (segment (start 135.636 52.324) (end 138.684 52.324) (width 0.254) (layer B.Cu) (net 14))
 (segment (start 138.684 52.324) (end 139.145 51.863) (width 0.254) (layer B.Cu) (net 14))
 (segment (start 139.145 51.863) (end 139.145 47.625) (width 0.254) (layer B.Cu) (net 14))
 (segment (start 128.905 53.34) (end 129.794 53.34) (width 0.254) (layer F.Cu) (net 15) (status 400000))
 (segment (start 162.005 46.689) (end 162.005 47.625) (width 0.254) (layer B.Cu) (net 15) (status 800000))
 (segment (start 160.528 45.212) (end 162.005 46.689) (width 0.254) (layer B.Cu) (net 15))
 (via (at 160.528 45.212) (size 0.6858) (drill 0.3302) (layers F.Cu B.Cu) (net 15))
 (segment (start 154.432 45.212) (end 160.528 45.212) (width 0.254) (layer F.Cu) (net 15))
 (segment (start 151.638 42.418) (end 154.432 45.212) (width 0.254) (layer F.Cu) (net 15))
 (segment (start 134.62 42.418) (end 151.638 42.418) (width 0.254) (layer F.Cu) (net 15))
 (segment (start 131.572 45.466) (end 134.62 42.418) (width 0.254) (layer F.Cu) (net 15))
 (segment (start 131.572 51.562) (end 131.572 45.466) (width 0.254) (layer F.Cu) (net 15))
 (segment (start 129.794 53.34) (end 131.572 51.562) (width 0.254) (layer F.Cu) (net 15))
 (segment (start 128.905 63.5) (end 118.11 63.5) (width 0.254) (layer F.Cu) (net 16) (status 400000))
 (segment (start 113.792 77.216) (end 113.792 78.058) (width 0.254) (layer B.Cu) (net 16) (status 800000))
 (segment (start 113.03 76.454) (end 113.792 77.216) (width 0.254) (layer B.Cu) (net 16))
 (segment (start 107.696 76.454) (end 113.03 76.454) (width 0.254) (layer B.Cu) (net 16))
 (segment (start 106.426 75.184) (end 107.696 76.454) (width 0.254) (layer B.Cu) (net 16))
 (via (at 106.426 75.184) (size 0.6858) (drill 0.3302) (layers F.Cu B.Cu) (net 16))
 (segment (start 118.11 63.5) (end 106.426 75.184) (width 0.254) (layer F.Cu) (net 16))
 (segment (start 113.792 78.058) (end 113.745 78.105) (width 0.254) (layer B.Cu) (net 16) (status C00000))
 (segment (start 144.145 68.58) (end 144.78 68.58) (width 0.254) (layer F.Cu) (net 17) (status C00000))
 (segment (start 144.78 68.58) (end 148.082 71.882) (width 0.254) (layer F.Cu) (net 17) (status 400000))
 (segment (start 148.082 71.882) (end 148.082 85.09) (width 0.254) (layer F.Cu) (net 17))
 (segment (start 148.082 85.09) (end 145.542 87.63) (width 0.254) (layer F.Cu) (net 17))
 (via (at 145.542 87.63) (size 0.6858) (drill 0.3302) (layers F.Cu B.Cu) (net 17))
 (segment (start 145.542 87.63) (end 141.732 83.82) (width 0.254) (layer B.Cu) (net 17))
 (segment (start 141.732 83.82) (end 139.145 83.82) (width 0.254) (layer B.Cu) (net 17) (status 800000))
 (segment (start 144.145 53.34) (end 144.145 53.467) (width 0.254) (layer F.Cu) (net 18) (status C00000))
 (segment (start 144.145 53.467) (end 147.066 56.388) (width 0.254) (layer F.Cu) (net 18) (status 400000))
 (segment (start 147.066 56.388) (end 147.066 58.42) (width 0.254) (layer F.Cu) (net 18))
 (segment (start 147.066 58.42) (end 156.21 67.564) (width 0.254) (layer F.Cu) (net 18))
 (segment (start 156.21 67.564) (end 156.21 76.708) (width 0.254) (layer F.Cu) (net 18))
 (via (at 156.21 76.708) (size 0.6858) (drill 0.3302) (layers F.Cu B.Cu) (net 18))
 (segment (start 156.21 76.708) (end 156.718 77.216) (width 0.254) (layer B.Cu) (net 18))
 (segment (start 156.718 77.216) (end 159.846 77.216) (width 0.254) (layer B.Cu) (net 18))
 (segment (start 159.846 77.216) (end 161.37 78.74) (width 0.254) (layer B.Cu) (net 18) (status 800000))
 (segment (start 128.905 68.58) (end 121.158 68.58) (width 0.254) (layer F.Cu) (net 19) (status 400000))
 (segment (start 114.554 109.22) (end 113.11 109.22) (width 0.254) (layer B.Cu) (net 19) (status 800000))
 (segment (start 114.808 108.966) (end 114.554 109.22) (width 0.254) (layer B.Cu) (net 19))
 (via (at 114.808 108.966) (size 0.6858) (drill 0.3302) (layers F.Cu B.Cu) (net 19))
 (segment (start 116.332 107.442) (end 114.808 108.966) (width 0.254) (layer F.Cu) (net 19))
 (segment (start 116.332 73.406) (end 116.332 107.442) (width 0.254) (layer F.Cu) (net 19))
 (segment (start 121.158 68.58) (end 116.332 73.406) (width 0.254) (layer F.Cu) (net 19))
 (segment (start 144.145 63.5) (end 144.78 63.5) (width 0.254) (layer F.Cu) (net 20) (status C00000))
 (segment (start 144.78 63.5) (end 150.622 69.342) (width 0.254) (layer F.Cu) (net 20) (status 400000))
 (segment (start 150.622 69.342) (end 150.622 87.63) (width 0.254) (layer F.Cu) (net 20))
 (segment (start 150.622 87.63) (end 141.478 96.774) (width 0.254) (layer F.Cu) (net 20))
 (segment (start 141.478 96.774) (end 135.128 96.774) (width 0.254) (layer F.Cu) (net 20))
 (segment (start 135.128 96.774) (end 133.096 98.806) (width 0.254) (layer F.Cu) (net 20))
 (segment (start 133.096 98.806) (end 133.096 108.966) (width 0.254) (layer F.Cu) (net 20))
 (via (at 133.096 108.966) (size 0.6858) (drill 0.3302) (layers F.Cu B.Cu) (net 20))
 (segment (start 133.096 108.966) (end 134.62 107.442) (width 0.254) (layer B.Cu) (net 20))
 (segment (start 134.62 107.442) (end 137.922 107.442) (width 0.254) (layer B.Cu) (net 20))
 (segment (start 137.922 107.442) (end 138.51 108.03) (width 0.254) (layer B.Cu) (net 20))
 (segment (start 138.51 108.03) (end 138.51 109.22) (width 0.254) (layer B.Cu) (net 20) (status 800000))
 (segment (start 144.145 58.42) (end 144.145 59.055) (width 0.254) (layer F.Cu) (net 21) (status C00000))
 (segment (start 144.145 59.055) (end 152.908 67.818) (width 0.254) (layer F.Cu) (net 21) (status 400000))
 (segment (start 152.908 67.818) (end 152.908 103.886) (width 0.254) (layer F.Cu) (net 21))
 (segment (start 152.908 103.886) (end 156.464 107.442) (width 0.254) (layer F.Cu) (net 21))
 (segment (start 156.464 107.442) (end 159.258 107.442) (width 0.254) (layer F.Cu) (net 21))
 (via (at 159.258 107.442) (size 0.6858) (drill 0.3302) (layers F.Cu B.Cu) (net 21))
 (segment (start 159.258 107.442) (end 161.036 107.442) (width 0.254) (layer B.Cu) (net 21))
 (segment (start 161.036 107.442) (end 161.37 107.776) (width 0.254) (layer B.Cu) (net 21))
 (segment (start 161.37 107.776) (end 161.37 109.22) (width 0.254) (layer B.Cu) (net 21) (status 800000))
 (segment (start 128.905 50.8) (end 119.634 50.8) (width 0.254) (layer F.Cu) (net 31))
 (segment (start 107.696 54.356) (end 106.68 55.372) (width 0.254) (layer F.Cu) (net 31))
 (segment (start 116.078 54.356) (end 107.696 54.356) (width 0.254) (layer F.Cu) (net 31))
 (segment (start 119.634 50.8) (end 116.078 54.356) (width 0.254) (layer F.Cu) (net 31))
 (segment (start 106.68 55.372) (end 106.68 55.88) (width 0.254) (layer F.Cu) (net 31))
 (segment (start 132.08 55.88) (end 132.08 57.404) (width 0.254) (layer F.Cu) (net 32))
 (segment (start 132.08 57.404) (end 128.905 60.579) (width 0.254) (layer F.Cu) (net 32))
 (segment (start 128.905 60.579) (end 128.905 60.96) (width 0.254) (layer F.Cu) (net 32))
 (segment (start 128.905 60.96) (end 128.905 60.579) (width 0.254) (layer F.Cu) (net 32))
 (segment (start 128.905 55.88) (end 129.286 55.88) (width 0.254) (layer F.Cu) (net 33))
 (segment (start 129.286 55.88) (end 132.842 52.324) (width 0.254) (layer F.Cu) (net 33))
 (segment (start 132.842 52.324) (end 132.842 45.466) (width 0.254) (layer F.Cu) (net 33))
 (segment (start 132.842 45.466) (end 134.62 43.688) (width 0.254) (layer F.Cu) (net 33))
 (segment (start 134.62 43.688) (end 150.876 43.688) (width 0.254) (layer F.Cu) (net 33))
 (segment (start 150.876 43.688) (end 154.94 47.752) (width 0.254) (layer F.Cu) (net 33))
 (segment (start 154.94 47.752) (end 154.94 55.88) (width 0.254) (layer F.Cu) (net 33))
 (segment (start 128.905 66.04) (end 118.11 66.04) (width 0.254) (layer F.Cu) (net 34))
 (segment (start 106.68 77.47) (end 106.68 86.36) (width 0.254) (layer F.Cu) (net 34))
 (segment (start 118.11 66.04) (end 106.68 77.47) (width 0.254) (layer F.Cu) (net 34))
 (segment (start 144.145 71.12) (end 145.034 71.12) (width 0.254) (layer F.Cu) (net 35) (status 400000))
 (segment (start 132.08 87.884) (end 132.08 86.36) (width 0.254) (layer F.Cu) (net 35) (status 800000))
 (segment (start 132.588 88.392) (end 132.08 87.884) (width 0.254) (layer F.Cu) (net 35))
 (segment (start 143.002 88.392) (end 132.588 88.392) (width 0.254) (layer F.Cu) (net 35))
 (segment (start 146.812 84.582) (end 143.002 88.392) (width 0.254) (layer F.Cu) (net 35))
 (segment (start 146.812 72.898) (end 146.812 84.582) (width 0.254) (layer F.Cu) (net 35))
 (segment (start 145.034 71.12) (end 146.812 72.898) (width 0.254) (layer F.Cu) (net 35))
 (segment (start 154.94 69.088) (end 154.94 68.072) (width 0.254) (layer F.Cu) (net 36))
 (segment (start 145.796 57.531) (end 144.145 55.88) (width 0.254) (layer F.Cu) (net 36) (status 800000))
 (segment (start 145.796 58.928) (end 145.796 57.531) (width 0.254) (layer F.Cu) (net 36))
 (segment (start 154.94 68.072) (end 145.796 58.928) (width 0.254) (layer F.Cu) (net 36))
 (segment (start 154.94 68.834) (end 154.94 69.088) (width 0.254) (layer F.Cu) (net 36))
 (segment (start 154.94 69.088) (end 154.94 89.662) (width 0.254) (layer F.Cu) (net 36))
 (segment (start 128.905 71.12) (end 122.174 71.12) (width 0.254) (layer F.Cu) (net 37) (status 400000))
 (segment (start 106.68 115.824) (end 106.68 116.84) (width 0.254) (layer F.Cu) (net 37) (status 800000))
 (segment (start 107.95 114.554) (end 106.68 115.824) (width 0.254) (layer F.Cu) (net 37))
 (segment (start 114.554 114.554) (end 107.95 114.554) (width 0.254) (layer F.Cu) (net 37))
 (segment (start 117.856 111.252) (end 114.554 114.554) (width 0.254) (layer F.Cu) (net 37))
 (segment (start 117.856 75.438) (end 117.856 111.252) (width 0.254) (layer F.Cu) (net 37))
 (segment (start 122.174 71.12) (end 117.856 75.438) (width 0.254) (layer F.Cu) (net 37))
 (segment (start 144.145 66.04) (end 145.034 66.04) (width 0.254) (layer F.Cu) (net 38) (status 400000))
 (segment (start 132.08 96.266) (end 132.08 116.84) (width 0.254) (layer F.Cu) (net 38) (status 800000))
 (segment (start 133.096 95.25) (end 132.08 96.266) (width 0.254) (layer F.Cu) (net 38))
 (segment (start 140.97 95.25) (end 133.096 95.25) (width 0.254) (layer F.Cu) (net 38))
 (segment (start 149.352 86.868) (end 140.97 95.25) (width 0.254) (layer F.Cu) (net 38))
 (segment (start 149.352 70.358) (end 149.352 86.868) (width 0.254) (layer F.Cu) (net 38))
 (segment (start 145.034 66.04) (end 149.352 70.358) (width 0.254) (layer F.Cu) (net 38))
 (segment (start 144.145 66.04) (end 144.78 66.04) (width 0.254) (layer F.Cu) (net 38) (status C00000))
 (segment (start 144.145 60.96) (end 144.526 60.96) (width 0.254) (layer F.Cu) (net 39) (status C00000))
 (segment (start 144.526 60.96) (end 151.638 68.072) (width 0.254) (layer F.Cu) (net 39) (status 400000))
 (segment (start 151.638 68.072) (end 151.638 115.57) (width 0.254) (layer F.Cu) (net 39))
 (segment (start 151.638 115.57) (end 152.908 116.84) (width 0.254) (layer F.Cu) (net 39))
 (segment (start 152.908 116.84) (end 154.94 116.84) (width 0.254) (layer F.Cu) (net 39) (status 800000)))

